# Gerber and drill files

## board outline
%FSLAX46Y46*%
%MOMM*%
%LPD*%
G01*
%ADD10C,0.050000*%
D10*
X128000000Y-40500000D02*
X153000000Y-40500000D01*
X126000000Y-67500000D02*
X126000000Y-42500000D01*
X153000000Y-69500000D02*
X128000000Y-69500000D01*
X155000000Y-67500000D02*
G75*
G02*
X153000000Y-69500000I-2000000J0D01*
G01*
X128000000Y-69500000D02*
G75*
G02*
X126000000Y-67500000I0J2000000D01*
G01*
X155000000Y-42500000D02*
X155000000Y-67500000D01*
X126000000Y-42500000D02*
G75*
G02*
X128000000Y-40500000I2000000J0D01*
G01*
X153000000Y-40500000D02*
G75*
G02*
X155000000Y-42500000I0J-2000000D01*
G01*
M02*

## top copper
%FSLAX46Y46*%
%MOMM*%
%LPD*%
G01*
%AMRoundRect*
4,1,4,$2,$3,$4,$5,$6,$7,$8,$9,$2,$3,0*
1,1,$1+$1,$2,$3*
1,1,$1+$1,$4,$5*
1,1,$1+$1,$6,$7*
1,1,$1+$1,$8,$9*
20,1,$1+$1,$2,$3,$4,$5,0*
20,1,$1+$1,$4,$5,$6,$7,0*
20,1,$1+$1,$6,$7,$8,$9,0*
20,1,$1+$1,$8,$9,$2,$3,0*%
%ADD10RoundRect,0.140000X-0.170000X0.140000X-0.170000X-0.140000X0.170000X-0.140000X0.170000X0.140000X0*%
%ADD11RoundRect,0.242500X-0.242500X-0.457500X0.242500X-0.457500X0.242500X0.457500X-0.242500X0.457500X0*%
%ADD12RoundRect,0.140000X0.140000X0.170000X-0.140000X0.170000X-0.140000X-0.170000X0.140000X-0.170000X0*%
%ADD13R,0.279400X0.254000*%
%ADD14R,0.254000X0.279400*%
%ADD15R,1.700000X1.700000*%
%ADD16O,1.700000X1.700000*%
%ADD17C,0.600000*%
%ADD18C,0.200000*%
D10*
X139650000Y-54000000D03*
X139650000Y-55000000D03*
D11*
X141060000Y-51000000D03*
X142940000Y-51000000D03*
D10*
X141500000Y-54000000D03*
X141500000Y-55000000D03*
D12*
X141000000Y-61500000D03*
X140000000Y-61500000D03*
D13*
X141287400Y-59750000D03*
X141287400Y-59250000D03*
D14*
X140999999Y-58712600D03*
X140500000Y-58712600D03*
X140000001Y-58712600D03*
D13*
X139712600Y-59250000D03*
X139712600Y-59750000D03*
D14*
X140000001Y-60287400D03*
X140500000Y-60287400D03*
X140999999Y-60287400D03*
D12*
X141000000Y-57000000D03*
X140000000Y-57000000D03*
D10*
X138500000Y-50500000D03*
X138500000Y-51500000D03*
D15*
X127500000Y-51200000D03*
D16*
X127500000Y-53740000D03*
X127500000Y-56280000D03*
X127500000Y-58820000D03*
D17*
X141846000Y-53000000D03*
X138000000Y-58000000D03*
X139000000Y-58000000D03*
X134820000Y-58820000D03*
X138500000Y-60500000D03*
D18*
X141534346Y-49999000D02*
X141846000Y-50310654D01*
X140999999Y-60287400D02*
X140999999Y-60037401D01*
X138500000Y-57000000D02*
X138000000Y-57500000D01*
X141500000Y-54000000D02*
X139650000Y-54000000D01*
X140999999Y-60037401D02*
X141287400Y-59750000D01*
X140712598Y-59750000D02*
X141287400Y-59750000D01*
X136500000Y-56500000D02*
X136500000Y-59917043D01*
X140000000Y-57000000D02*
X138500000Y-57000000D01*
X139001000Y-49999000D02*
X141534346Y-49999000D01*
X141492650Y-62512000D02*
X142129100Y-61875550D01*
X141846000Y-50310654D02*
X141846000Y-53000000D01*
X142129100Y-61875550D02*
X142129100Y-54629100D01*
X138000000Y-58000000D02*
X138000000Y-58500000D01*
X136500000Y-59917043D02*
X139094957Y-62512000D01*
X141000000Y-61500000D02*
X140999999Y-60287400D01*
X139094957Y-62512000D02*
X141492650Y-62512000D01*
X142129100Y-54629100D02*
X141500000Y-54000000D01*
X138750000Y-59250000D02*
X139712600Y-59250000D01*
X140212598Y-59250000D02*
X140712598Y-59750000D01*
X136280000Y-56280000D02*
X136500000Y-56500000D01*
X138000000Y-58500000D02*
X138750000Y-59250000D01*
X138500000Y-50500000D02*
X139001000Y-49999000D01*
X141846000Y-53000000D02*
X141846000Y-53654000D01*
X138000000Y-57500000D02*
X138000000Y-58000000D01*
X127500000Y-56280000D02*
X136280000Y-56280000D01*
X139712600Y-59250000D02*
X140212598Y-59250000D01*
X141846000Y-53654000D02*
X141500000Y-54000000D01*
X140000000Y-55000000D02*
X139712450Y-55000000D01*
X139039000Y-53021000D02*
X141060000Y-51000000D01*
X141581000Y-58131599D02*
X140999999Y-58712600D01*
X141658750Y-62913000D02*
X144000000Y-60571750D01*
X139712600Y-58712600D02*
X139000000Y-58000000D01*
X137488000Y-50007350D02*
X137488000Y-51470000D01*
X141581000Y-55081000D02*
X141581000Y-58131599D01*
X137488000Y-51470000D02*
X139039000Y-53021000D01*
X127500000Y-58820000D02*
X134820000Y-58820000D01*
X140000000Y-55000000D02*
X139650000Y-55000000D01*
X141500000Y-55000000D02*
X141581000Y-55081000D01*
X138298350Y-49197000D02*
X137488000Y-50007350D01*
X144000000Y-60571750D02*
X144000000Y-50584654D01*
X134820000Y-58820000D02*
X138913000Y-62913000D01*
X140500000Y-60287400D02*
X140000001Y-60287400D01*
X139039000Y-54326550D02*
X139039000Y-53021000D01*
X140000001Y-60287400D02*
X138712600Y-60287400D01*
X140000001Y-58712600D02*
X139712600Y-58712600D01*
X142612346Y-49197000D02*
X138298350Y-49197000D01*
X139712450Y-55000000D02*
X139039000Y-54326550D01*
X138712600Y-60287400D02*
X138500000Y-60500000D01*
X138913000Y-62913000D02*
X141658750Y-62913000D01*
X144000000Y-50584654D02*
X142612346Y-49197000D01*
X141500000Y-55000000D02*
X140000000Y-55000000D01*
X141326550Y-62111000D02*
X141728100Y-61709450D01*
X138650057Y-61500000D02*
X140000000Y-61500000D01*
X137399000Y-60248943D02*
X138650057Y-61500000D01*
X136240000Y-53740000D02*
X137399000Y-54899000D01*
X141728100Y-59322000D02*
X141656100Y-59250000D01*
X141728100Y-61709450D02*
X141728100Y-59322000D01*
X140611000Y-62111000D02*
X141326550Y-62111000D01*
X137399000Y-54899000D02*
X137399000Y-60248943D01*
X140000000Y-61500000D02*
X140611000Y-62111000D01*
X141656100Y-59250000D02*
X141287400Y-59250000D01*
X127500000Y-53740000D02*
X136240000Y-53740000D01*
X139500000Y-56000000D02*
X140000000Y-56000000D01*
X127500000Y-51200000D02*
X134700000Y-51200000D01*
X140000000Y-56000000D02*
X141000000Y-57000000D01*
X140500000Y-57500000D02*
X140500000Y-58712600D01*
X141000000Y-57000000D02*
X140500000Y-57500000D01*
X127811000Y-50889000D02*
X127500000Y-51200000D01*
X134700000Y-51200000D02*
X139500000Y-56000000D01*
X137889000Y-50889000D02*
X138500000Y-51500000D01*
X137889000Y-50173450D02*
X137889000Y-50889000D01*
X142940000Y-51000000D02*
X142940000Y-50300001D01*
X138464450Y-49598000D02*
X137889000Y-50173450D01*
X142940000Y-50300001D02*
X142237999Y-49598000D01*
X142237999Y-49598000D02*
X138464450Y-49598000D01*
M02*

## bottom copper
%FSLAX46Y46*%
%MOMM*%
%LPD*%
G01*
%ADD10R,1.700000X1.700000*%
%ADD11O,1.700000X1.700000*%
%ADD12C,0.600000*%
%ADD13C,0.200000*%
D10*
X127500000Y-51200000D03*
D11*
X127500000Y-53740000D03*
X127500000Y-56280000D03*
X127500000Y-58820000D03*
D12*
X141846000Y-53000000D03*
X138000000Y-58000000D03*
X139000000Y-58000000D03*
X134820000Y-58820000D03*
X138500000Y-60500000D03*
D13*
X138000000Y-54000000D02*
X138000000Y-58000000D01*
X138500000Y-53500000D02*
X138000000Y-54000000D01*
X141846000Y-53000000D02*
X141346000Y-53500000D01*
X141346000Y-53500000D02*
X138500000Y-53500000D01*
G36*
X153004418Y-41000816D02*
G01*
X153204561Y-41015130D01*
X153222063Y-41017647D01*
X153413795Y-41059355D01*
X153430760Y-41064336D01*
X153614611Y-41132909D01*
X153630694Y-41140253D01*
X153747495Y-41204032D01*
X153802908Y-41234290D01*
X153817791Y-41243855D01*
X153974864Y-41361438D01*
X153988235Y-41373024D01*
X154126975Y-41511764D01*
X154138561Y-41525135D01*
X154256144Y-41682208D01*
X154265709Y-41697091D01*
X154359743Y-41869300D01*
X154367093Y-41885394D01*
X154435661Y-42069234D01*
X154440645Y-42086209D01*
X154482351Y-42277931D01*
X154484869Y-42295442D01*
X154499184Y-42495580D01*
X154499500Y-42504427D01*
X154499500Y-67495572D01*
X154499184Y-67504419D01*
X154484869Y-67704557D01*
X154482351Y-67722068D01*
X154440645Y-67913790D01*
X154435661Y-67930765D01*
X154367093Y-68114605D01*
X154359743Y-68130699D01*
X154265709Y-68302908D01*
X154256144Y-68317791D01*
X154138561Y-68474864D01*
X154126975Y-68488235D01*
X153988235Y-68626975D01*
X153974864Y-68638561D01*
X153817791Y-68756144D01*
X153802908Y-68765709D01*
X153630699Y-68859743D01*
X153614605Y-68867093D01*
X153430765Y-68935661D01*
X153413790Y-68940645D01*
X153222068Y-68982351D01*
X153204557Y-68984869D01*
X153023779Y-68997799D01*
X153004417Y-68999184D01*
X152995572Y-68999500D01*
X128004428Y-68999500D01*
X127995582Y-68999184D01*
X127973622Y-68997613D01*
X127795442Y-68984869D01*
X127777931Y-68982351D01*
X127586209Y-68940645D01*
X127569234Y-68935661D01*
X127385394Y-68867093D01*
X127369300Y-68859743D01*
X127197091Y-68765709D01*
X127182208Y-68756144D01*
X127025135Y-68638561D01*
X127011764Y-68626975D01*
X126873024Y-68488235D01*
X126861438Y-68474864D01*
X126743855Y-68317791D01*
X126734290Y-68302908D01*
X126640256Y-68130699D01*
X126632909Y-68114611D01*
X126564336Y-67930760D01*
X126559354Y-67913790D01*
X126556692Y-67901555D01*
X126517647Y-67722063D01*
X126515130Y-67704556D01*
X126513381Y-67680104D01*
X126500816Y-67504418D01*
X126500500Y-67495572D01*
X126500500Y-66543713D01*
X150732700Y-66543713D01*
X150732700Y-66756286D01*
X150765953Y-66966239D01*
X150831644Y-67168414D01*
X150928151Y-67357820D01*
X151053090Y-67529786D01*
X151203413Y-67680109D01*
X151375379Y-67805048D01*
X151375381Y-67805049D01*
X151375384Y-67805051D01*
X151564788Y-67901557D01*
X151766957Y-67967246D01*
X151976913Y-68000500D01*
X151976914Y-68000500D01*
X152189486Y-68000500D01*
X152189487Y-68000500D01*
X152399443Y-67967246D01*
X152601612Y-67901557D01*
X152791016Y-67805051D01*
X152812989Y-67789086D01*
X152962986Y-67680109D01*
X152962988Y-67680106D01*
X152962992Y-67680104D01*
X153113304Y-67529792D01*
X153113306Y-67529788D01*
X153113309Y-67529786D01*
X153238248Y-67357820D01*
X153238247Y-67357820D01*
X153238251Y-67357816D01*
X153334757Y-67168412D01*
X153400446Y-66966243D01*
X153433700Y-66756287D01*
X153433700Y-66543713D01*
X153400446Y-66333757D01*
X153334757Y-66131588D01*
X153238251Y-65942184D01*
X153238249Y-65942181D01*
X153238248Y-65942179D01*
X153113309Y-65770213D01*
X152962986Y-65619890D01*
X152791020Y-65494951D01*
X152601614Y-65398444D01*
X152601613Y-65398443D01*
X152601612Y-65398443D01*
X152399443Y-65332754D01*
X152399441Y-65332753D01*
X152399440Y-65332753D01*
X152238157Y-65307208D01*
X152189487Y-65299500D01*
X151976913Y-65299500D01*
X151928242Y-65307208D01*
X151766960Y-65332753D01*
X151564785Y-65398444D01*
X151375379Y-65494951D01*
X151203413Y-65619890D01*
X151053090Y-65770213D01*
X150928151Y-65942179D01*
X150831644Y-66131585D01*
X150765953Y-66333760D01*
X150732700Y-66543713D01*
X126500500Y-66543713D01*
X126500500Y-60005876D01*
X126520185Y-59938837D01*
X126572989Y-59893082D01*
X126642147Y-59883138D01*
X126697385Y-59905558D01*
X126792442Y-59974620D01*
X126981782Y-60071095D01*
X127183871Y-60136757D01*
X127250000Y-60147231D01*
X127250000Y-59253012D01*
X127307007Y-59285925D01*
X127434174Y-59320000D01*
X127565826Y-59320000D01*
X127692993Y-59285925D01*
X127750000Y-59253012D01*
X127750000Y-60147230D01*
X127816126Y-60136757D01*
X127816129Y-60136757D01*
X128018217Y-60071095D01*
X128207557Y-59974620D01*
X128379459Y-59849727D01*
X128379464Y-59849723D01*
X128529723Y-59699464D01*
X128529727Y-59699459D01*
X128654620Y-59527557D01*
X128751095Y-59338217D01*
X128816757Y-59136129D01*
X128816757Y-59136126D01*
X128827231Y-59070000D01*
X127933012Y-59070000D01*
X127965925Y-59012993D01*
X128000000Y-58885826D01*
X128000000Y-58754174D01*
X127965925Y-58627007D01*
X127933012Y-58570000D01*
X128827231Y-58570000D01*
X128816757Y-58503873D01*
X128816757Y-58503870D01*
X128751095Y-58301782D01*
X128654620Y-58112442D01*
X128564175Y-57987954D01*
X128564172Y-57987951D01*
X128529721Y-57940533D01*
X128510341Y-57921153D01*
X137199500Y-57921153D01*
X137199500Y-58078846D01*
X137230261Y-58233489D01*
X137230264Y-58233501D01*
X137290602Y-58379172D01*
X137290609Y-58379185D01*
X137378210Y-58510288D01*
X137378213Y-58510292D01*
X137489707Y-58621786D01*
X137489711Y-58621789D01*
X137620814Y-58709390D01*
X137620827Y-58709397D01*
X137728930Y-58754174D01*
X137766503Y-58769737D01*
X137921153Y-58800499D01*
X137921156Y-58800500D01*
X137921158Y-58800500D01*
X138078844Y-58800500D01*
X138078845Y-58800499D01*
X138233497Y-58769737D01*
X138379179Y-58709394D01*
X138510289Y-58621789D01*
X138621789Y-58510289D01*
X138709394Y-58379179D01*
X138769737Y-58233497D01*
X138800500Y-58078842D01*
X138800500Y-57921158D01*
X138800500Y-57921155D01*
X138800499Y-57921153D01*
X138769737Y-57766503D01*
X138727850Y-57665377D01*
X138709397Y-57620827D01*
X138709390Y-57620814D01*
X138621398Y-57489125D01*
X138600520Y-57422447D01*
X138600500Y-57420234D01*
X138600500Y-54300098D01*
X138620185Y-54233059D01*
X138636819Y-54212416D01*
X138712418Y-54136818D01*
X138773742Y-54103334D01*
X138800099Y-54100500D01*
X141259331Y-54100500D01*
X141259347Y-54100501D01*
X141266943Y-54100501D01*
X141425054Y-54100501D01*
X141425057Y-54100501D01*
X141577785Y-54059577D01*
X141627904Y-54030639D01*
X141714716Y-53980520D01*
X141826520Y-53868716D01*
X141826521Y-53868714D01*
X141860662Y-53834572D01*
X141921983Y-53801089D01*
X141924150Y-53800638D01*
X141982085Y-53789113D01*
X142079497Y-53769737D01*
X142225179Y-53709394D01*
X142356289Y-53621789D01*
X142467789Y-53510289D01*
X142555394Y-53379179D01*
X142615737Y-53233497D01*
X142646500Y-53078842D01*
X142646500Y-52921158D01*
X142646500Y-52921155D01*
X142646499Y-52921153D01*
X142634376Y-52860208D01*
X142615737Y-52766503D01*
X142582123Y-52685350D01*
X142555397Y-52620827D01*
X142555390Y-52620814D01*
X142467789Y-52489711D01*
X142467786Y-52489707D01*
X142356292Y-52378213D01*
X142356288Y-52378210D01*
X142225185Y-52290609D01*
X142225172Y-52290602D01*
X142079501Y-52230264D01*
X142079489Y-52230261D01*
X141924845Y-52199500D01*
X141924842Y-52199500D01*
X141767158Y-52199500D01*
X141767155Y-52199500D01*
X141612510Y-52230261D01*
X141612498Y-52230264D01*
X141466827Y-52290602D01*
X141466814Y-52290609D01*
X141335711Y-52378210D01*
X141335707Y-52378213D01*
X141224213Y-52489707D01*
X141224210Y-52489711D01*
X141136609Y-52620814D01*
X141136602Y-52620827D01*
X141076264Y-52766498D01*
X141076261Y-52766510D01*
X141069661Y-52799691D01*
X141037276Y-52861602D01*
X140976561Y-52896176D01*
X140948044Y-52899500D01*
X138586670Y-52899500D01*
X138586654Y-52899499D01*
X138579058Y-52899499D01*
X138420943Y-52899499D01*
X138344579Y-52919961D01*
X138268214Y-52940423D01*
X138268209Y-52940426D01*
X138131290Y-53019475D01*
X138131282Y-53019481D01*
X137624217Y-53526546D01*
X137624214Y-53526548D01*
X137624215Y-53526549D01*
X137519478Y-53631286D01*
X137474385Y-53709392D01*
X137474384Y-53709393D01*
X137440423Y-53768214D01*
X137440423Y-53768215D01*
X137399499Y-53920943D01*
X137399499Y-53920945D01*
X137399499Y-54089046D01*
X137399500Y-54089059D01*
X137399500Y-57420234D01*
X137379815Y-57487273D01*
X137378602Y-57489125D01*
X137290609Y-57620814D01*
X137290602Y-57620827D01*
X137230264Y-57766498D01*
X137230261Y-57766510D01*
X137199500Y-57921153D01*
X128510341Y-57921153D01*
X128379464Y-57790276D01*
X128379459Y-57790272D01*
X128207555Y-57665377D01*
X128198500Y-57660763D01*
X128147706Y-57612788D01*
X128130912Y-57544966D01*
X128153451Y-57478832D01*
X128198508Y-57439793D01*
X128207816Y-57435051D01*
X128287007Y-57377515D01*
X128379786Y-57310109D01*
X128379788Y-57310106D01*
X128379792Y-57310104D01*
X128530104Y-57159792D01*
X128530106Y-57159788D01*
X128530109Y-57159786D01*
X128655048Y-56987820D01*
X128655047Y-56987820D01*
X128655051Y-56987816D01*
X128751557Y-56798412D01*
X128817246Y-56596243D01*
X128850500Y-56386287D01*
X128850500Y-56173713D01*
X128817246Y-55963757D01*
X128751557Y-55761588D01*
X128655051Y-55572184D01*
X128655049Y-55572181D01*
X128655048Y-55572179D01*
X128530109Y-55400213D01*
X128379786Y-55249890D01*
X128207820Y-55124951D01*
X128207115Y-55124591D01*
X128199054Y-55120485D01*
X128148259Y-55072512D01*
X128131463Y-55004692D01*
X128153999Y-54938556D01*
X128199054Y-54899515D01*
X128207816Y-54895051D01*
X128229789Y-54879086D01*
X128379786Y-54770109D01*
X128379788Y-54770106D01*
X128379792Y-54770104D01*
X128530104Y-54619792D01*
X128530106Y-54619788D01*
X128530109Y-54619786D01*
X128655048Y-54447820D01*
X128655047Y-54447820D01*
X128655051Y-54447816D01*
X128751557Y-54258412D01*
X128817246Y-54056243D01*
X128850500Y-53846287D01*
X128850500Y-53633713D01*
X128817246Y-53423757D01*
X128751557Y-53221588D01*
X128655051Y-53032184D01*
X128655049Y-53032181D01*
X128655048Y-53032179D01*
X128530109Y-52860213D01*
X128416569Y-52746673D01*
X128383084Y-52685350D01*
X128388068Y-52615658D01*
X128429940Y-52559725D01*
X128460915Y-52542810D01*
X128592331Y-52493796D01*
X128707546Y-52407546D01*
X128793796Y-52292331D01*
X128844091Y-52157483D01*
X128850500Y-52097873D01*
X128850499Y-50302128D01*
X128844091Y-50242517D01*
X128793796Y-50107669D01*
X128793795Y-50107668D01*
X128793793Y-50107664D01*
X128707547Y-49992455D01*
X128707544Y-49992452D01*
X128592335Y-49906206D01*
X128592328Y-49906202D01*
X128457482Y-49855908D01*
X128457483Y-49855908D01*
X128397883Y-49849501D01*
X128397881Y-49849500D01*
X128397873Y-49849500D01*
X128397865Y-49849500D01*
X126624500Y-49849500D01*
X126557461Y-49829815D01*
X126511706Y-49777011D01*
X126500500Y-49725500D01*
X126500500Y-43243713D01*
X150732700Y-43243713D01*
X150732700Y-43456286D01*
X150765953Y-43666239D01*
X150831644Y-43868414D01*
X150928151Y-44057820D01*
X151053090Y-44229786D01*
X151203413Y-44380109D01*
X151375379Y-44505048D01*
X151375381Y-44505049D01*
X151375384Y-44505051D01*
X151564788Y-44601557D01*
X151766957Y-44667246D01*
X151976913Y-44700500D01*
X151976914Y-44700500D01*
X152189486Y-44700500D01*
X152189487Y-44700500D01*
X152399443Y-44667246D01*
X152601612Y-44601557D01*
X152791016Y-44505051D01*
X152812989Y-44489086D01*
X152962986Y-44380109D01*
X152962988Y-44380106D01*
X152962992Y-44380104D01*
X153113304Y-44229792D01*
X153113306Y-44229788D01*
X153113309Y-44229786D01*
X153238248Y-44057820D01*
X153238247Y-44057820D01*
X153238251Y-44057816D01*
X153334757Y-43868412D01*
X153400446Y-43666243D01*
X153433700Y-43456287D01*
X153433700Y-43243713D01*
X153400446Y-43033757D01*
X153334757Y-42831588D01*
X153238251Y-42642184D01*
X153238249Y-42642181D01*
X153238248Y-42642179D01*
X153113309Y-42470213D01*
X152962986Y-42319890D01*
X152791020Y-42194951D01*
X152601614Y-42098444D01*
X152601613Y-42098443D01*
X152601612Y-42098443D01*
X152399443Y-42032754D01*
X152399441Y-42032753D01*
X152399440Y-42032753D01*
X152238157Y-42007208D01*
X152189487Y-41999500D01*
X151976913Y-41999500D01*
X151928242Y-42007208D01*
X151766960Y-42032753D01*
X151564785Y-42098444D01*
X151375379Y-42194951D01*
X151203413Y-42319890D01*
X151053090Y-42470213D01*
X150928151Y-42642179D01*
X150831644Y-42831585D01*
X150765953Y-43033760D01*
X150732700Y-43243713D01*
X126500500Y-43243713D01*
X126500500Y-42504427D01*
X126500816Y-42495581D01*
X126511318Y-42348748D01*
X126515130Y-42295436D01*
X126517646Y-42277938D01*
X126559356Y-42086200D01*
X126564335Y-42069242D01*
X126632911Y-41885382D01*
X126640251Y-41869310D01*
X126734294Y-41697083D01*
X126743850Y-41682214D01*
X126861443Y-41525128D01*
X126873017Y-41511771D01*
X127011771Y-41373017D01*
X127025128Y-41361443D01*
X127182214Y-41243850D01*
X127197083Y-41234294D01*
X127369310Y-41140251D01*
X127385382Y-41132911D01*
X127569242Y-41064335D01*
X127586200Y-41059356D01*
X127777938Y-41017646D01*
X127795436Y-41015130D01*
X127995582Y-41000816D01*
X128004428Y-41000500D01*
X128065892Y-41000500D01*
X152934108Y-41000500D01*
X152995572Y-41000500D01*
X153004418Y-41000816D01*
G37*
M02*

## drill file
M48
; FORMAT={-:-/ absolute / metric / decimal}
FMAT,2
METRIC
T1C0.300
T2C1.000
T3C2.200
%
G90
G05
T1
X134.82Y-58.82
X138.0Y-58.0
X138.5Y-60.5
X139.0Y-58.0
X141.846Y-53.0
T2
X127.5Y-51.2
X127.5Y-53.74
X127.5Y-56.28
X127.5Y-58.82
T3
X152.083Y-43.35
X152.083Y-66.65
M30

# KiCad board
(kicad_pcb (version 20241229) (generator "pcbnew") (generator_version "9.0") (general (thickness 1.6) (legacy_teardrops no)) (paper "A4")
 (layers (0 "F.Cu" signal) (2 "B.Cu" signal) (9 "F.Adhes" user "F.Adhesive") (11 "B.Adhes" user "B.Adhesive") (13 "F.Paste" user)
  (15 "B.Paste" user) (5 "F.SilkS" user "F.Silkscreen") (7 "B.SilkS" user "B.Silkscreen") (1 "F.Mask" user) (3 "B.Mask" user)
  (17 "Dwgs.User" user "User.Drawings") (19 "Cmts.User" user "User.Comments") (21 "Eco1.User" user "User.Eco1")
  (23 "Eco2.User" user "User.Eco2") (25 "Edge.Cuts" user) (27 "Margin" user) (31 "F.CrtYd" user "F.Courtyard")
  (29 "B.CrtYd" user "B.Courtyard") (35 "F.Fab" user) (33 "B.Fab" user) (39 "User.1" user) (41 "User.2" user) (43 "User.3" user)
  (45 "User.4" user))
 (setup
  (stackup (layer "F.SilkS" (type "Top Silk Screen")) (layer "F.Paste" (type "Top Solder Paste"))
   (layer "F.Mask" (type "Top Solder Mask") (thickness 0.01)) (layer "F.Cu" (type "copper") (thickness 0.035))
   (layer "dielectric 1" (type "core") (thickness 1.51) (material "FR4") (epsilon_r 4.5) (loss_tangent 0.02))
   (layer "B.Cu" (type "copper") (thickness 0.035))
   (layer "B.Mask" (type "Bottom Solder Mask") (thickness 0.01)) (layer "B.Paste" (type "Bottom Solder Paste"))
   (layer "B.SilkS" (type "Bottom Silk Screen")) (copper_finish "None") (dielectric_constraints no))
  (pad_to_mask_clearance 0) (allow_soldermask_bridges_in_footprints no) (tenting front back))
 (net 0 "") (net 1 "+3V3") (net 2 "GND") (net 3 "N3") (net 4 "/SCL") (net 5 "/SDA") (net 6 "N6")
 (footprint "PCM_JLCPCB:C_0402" (layer "F.Cu") (at 139.65 54.5 -90)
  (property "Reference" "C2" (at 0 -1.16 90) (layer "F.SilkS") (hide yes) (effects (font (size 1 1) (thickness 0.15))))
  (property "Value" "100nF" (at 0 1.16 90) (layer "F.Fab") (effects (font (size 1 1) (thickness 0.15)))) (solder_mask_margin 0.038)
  (pad "1" smd roundrect (at -0.5 0 270) (size 0.56 0.62) (layers "F.Cu" "F.Mask" "F.Paste") (roundrect_rratio 0.25) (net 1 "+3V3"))
  (pad "2" smd roundrect (at 0.5 0 270) (size 0.56 0.62) (layers "F.Cu" "F.Mask" "F.Paste") (roundrect_rratio 0.25) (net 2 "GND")))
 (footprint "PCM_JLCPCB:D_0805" (layer "F.Cu") (at 142 51)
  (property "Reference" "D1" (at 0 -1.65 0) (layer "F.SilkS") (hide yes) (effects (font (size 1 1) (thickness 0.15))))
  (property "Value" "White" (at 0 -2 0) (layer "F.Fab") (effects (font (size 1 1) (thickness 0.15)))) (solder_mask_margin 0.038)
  (pad "1" smd roundrect (at -0.94 0) (size 0.97 1.4) (layers "F.Cu" "F.Mask" "F.Paste") (roundrect_rratio 0.25) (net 2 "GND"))
  (pad "2" smd roundrect (at 0.94 0) (size 0.97 1.4) (layers "F.Cu" "F.Mask" "F.Paste") (roundrect_rratio 0.25) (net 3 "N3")))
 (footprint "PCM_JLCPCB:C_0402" (layer "F.Cu") (at 141.5 54.5 -90)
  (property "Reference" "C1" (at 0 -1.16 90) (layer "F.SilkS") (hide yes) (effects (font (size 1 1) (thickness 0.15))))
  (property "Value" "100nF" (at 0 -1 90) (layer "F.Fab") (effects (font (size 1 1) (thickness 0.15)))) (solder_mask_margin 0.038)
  (pad "1" smd roundrect (at -0.5 0 270) (size 0.56 0.62) (layers "F.Cu" "F.Mask" "F.Paste") (roundrect_rratio 0.25) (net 1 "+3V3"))
  (pad "2" smd roundrect (at 0.5 0 270) (size 0.56 0.62) (layers "F.Cu" "F.Mask" "F.Paste") (roundrect_rratio 0.25) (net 2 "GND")))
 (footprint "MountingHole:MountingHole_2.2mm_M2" (layer "F.Cu") (at 152.0832 66.65)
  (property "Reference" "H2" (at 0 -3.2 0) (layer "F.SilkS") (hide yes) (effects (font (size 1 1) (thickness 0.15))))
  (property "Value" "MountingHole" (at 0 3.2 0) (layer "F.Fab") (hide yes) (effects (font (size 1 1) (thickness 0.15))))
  (pad "" np_thru_hole circle (at 0 0) (size 2.2 2.2) (drill 2.2) (layers "*.Cu" "*.Mask")))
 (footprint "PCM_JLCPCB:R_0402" (layer "F.Cu") (at 140.5 61.5 180)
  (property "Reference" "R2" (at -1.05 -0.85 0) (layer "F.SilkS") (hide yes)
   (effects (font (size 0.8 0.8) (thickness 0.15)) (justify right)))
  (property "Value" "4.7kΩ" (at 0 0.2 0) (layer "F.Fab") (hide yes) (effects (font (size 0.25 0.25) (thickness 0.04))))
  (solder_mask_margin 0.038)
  (pad "1" smd roundrect (at -0.5 0 180) (size 0.56 0.62) (layers "F.Cu" "F.Mask" "F.Paste") (roundrect_rratio 0.25) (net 1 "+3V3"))
  (pad "2" smd roundrect (at 0.5 0 180) (size 0.56 0.62) (layers "F.Cu" "F.Mask" "F.Paste") (roundrect_rratio 0.25) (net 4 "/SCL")))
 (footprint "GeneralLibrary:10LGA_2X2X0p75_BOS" (layer "F.Cu") (at 140.5 59.5 180)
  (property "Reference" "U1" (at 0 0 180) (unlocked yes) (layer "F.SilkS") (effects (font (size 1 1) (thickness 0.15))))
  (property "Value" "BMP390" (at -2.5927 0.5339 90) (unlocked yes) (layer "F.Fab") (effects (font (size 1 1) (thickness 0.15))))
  (pad "1" smd rect (at -0.7874 -0.25 270) (size 0.254 0.2794) (layers "F.Cu" "F.Mask" "F.Paste") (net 1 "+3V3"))
  (pad "2" smd rect (at -0.7874 0.25 270) (size 0.254 0.2794) (layers "F.Cu" "F.Mask" "F.Paste") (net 4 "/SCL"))
  (pad "3" smd rect (at -0.499999 0.7874 180) (size 0.254 0.2794) (layers "F.Cu" "F.Mask" "F.Paste") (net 2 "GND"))
  (pad "4" smd rect (at 0 0.7874 180) (size 0.254 0.2794) (layers "F.Cu" "F.Mask" "F.Paste") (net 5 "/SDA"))
  (pad "5" smd rect (at 0.499999 0.7874 180) (size 0.254 0.2794) (layers "F.Cu" "F.Mask" "F.Paste") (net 2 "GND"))
  (pad "6" smd rect (at 0.7874 0.25 270) (size 0.254 0.2794) (layers "F.Cu" "F.Mask" "F.Paste") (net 1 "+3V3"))
  (pad "7" smd rect (at 0.7874 -0.25 270) (size 0.254 0.2794) (layers "F.Cu" "F.Mask" "F.Paste") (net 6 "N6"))
  (pad "8" smd rect (at 0.499999 -0.7874 180) (size 0.254 0.2794) (layers "F.Cu" "F.Mask" "F.Paste") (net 2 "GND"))
  (pad "9" smd rect (at 0 -0.7874 180) (size 0.254 0.2794) (layers "F.Cu" "F.Mask" "F.Paste") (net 2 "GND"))
  (pad "10" smd rect (at -0.499999 -0.7874 180) (size 0.254 0.2794) (layers "F.Cu" "F.Mask" "F.Paste") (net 1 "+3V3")))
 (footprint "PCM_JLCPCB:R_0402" (layer "F.Cu") (at 140.5 57 180)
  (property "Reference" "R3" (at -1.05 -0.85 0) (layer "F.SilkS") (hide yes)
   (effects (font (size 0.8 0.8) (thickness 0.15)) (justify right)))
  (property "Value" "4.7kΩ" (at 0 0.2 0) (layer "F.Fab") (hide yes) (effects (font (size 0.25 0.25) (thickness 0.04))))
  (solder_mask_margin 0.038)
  (pad "1" smd roundrect (at -0.5 0 180) (size 0.56 0.62) (layers "F.Cu" "F.Mask" "F.Paste") (roundrect_rratio 0.25) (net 5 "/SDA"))
  (pad "2" smd roundrect (at 0.5 0 180) (size 0.56 0.62) (layers "F.Cu" "F.Mask" "F.Paste") (roundrect_rratio 0.25) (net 1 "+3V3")))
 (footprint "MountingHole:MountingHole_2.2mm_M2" (layer "F.Cu") (at 152.0832 43.35)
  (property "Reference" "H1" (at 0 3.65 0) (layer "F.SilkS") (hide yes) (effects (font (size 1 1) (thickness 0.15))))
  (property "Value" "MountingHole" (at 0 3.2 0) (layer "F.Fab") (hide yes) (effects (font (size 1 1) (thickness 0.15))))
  (pad "" np_thru_hole circle (at 0 0) (size 2.2 2.2) (drill 2.2) (layers "*.Cu" "*.Mask")))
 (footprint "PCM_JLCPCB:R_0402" (layer "F.Cu") (at 138.5 51 -90)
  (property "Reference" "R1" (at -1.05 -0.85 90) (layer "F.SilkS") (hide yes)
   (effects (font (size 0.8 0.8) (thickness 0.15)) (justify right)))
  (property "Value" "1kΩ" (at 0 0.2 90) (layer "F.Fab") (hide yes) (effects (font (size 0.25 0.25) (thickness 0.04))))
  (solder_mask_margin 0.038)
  (pad "1" smd roundrect (at -0.5 0 270) (size 0.56 0.62) (layers "F.Cu" "F.Mask" "F.Paste") (roundrect_rratio 0.25) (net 1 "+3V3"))
  (pad "2" smd roundrect (at 0.5 0 270) (size 0.56 0.62) (layers "F.Cu" "F.Mask" "F.Paste") (roundrect_rratio 0.25) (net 3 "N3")))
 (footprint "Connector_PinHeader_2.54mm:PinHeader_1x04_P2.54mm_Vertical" (layer "B.Cu") (at 127.5 51.2 180)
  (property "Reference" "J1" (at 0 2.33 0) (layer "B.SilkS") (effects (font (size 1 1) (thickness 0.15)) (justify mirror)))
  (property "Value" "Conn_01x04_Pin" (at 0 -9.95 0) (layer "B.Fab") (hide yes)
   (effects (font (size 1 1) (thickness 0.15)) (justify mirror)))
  (pad "1" thru_hole rect (at 0 0 180) (size 1.7 1.7) (drill 1) (layers "*.Cu" "*.Mask") (remove_unused_layers no) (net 5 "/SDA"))
  (pad "2" thru_hole oval (at 0 -2.54 180) (size 1.7 1.7) (drill 1) (layers "*.Cu" "*.Mask") (remove_unused_layers no) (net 4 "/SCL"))
  (pad "3" thru_hole oval (at 0 -5.08 180) (size 1.7 1.7) (drill 1) (layers "*.Cu" "*.Mask") (remove_unused_layers no) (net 1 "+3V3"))
  (pad "4" thru_hole oval (at 0 -7.62 180) (size 1.7 1.7) (drill 1) (layers "*.Cu" "*.Mask") (remove_unused_layers no) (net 2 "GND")))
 (gr_line (start 128 40.5) (end 153 40.5) (stroke (width 0.05) (type default)) (layer "Edge.Cuts"))
 (gr_line (start 126 67.5) (end 126 42.5) (stroke (width 0.05) (type default)) (layer "Edge.Cuts"))
 (gr_line (start 153 69.5) (end 128 69.5) (stroke (width 0.05) (type default)) (layer "Edge.Cuts"))
 (gr_arc (start 155 67.5) (mid 154.414214 68.914214) (end 153 69.5) (stroke (width 0.05) (type default)) (layer "Edge.Cuts"))
 (gr_arc (start 128 69.5) (mid 126.585786 68.914214) (end 126 67.5) (stroke (width 0.05) (type default)) (layer "Edge.Cuts"))
 (gr_line (start 155 42.5) (end 155 67.5) (stroke (width 0.05) (type default)) (layer "Edge.Cuts"))
 (gr_arc (start 126 42.5) (mid 126.585786 41.085786) (end 128 40.5) (stroke (width 0.05) (type default)) (layer "Edge.Cuts"))
 (gr_arc (start 153 40.5) (mid 154.414214 41.085786) (end 155 42.5) (stroke (width 0.05) (type default)) (layer "Edge.Cuts"))
 (segment (start 141.534346 49.999) (end 141.846 50.310654) (width 0.2) (layer "F.Cu") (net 1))
 (segment (start 140.999999 60.2874) (end 140.999999 60.037401) (width 0.2) (layer "F.Cu") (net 1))
 (segment (start 138.5 57) (end 138 57.5) (width 0.2) (layer "F.Cu") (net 1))
 (segment (start 141.5 54) (end 139.65 54) (width 0.2) (layer "F.Cu") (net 1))
 (segment (start 140.999999 60.037401) (end 141.2874 59.75) (width 0.2) (layer "F.Cu") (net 1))
 (segment (start 140.712598 59.75) (end 141.2874 59.75) (width 0.2) (layer "F.Cu") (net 1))
 (segment (start 136.5 56.5) (end 136.5 59.917043) (width 0.2) (layer "F.Cu") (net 1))
 (segment (start 140 57) (end 138.5 57) (width 0.2) (layer "F.Cu") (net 1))
 (segment (start 139.001 49.999) (end 141.534346 49.999) (width 0.2) (layer "F.Cu") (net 1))
 (segment (start 141.49265 62.512) (end 142.1291 61.87555) (width 0.2) (layer "F.Cu") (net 1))
 (segment (start 141.846 50.310654) (end 141.846 53) (width 0.2) (layer "F.Cu") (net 1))
 (segment (start 142.1291 61.87555) (end 142.1291 54.6291) (width 0.2) (layer "F.Cu") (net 1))
 (segment (start 138 58) (end 138 58.5) (width 0.2) (layer "F.Cu") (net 1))
 (segment (start 136.5 59.917043) (end 139.094957 62.512) (width 0.2) (layer "F.Cu") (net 1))
 (segment (start 141 61.5) (end 140.999999 60.2874) (width 0.2) (layer "F.Cu") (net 1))
 (segment (start 139.094957 62.512) (end 141.49265 62.512) (width 0.2) (layer "F.Cu") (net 1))
 (segment (start 142.1291 54.6291) (end 141.5 54) (width 0.2) (layer "F.Cu") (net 1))
 (segment (start 138.75 59.25) (end 139.7126 59.25) (width 0.2) (layer "F.Cu") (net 1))
 (segment (start 140.212598 59.25) (end 140.712598 59.75) (width 0.2) (layer "F.Cu") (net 1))
 (segment (start 136.28 56.28) (end 136.5 56.5) (width 0.2) (layer "F.Cu") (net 1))
 (segment (start 138 58.5) (end 138.75 59.25) (width 0.2) (layer "F.Cu") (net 1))
 (segment (start 138.5 50.5) (end 139.001 49.999) (width 0.2) (layer "F.Cu") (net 1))
 (segment (start 141.846 53) (end 141.846 53.654) (width 0.2) (layer "F.Cu") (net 1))
 (segment (start 138 57.5) (end 138 58) (width 0.2) (layer "F.Cu") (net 1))
 (segment (start 127.5 56.28) (end 136.28 56.28) (width 0.2) (layer "F.Cu") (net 1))
 (segment (start 139.7126 59.25) (end 140.212598 59.25) (width 0.2) (layer "F.Cu") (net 1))
 (segment (start 141.846 53.654) (end 141.5 54) (width 0.2) (layer "F.Cu") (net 1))
 (via (at 141.846 53) (size 0.6) (drill 0.3) (layers "F.Cu" "B.Cu") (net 1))
 (via (at 138 58) (size 0.6) (drill 0.3) (layers "F.Cu" "B.Cu") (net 1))
 (segment (start 138 54) (end 138 58) (width 0.2) (layer "B.Cu") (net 1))
 (segment (start 138.5 53.5) (end 138 54) (width 0.2) (layer "B.Cu") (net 1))
 (segment (start 141.846 53) (end 141.346 53.5) (width 0.2) (layer "B.Cu") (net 1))
 (segment (start 141.346 53.5) (end 138.5 53.5) (width 0.2) (layer "B.Cu") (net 1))
 (segment (start 140 55) (end 139.71245 55) (width 0.2) (layer "F.Cu") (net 2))
 (segment (start 139.039 53.021) (end 141.06 51) (width 0.2) (layer "F.Cu") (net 2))
 (segment (start 141.581 58.131599) (end 140.999999 58.7126) (width 0.2) (layer "F.Cu") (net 2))
 (segment (start 141.65875 62.913) (end 144 60.57175) (width 0.2) (layer "F.Cu") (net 2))
 (segment (start 139.7126 58.7126) (end 139 58) (width 0.2) (layer "F.Cu") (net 2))
 (segment (start 137.488 50.00735) (end 137.488 51.47) (width 0.2) (layer "F.Cu") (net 2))
 (segment (start 141.581 55.081) (end 141.581 58.131599) (width 0.2) (layer "F.Cu") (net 2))
 (segment (start 137.488 51.47) (end 139.039 53.021) (width 0.2) (layer "F.Cu") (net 2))
 (segment (start 127.5 58.82) (end 134.82 58.82) (width 0.2) (layer "F.Cu") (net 2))
 (segment (start 140 55) (end 139.65 55) (width 0.2) (layer "F.Cu") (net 2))
 (segment (start 141.5 55) (end 141.581 55.081) (width 0.2) (layer "F.Cu") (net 2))
 (segment (start 138.29835 49.197) (end 137.488 50.00735) (width 0.2) (layer "F.Cu") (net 2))
 (segment (start 144 60.57175) (end 144 50.584654) (width 0.2) (layer "F.Cu") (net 2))
 (segment (start 134.82 58.82) (end 138.913 62.913) (width 0.2) (layer "F.Cu") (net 2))
 (segment (start 140.5 60.2874) (end 140.000001 60.2874) (width 0.2) (layer "F.Cu") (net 2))
 (segment (start 139.039 54.32655) (end 139.039 53.021) (width 0.2) (layer "F.Cu") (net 2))
 (segment (start 140.000001 60.2874) (end 138.7126 60.2874) (width 0.2) (layer "F.Cu") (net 2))
 (segment (start 140.000001 58.7126) (end 139.7126 58.7126) (width 0.2) (layer "F.Cu") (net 2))
 (segment (start 142.612346 49.197) (end 138.29835 49.197) (width 0.2) (layer "F.Cu") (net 2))
 (segment (start 139.71245 55) (end 139.039 54.32655) (width 0.2) (layer "F.Cu") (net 2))
 (segment (start 138.7126 60.2874) (end 138.5 60.5) (width 0.2) (layer "F.Cu") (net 2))
 (segment (start 138.913 62.913) (end 141.65875 62.913) (width 0.2) (layer "F.Cu") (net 2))
 (segment (start 144 50.584654) (end 142.612346 49.197) (width 0.2) (layer "F.Cu") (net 2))
 (segment (start 141.5 55) (end 140 55) (width 0.2) (layer "F.Cu") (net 2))
 (via (at 139 58) (size 0.6) (drill 0.3) (layers "F.Cu" "B.Cu") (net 2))
 (via (at 134.82 58.82) (size 0.6) (drill 0.3) (layers "F.Cu" "B.Cu") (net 2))
 (via (at 138.5 60.5) (size 0.6) (drill 0.3) (layers "F.Cu" "B.Cu") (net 2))
 (segment (start 141.32655 62.111) (end 141.7281 61.70945) (width 0.2) (layer "F.Cu") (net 4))
 (segment (start 138.650057 61.5) (end 140 61.5) (width 0.2) (layer "F.Cu") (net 4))
 (segment (start 137.399 60.248943) (end 138.650057 61.5) (width 0.2) (layer "F.Cu") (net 4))
 (segment (start 136.24 53.74) (end 137.399 54.899) (width 0.2) (layer "F.Cu") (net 4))
 (segment (start 141.7281 59.322) (end 141.6561 59.25) (width 0.2) (layer "F.Cu") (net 4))
 (segment (start 141.7281 61.70945) (end 141.7281 59.322) (width 0.2) (layer "F.Cu") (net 4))
 (segment (start 140.611 62.111) (end 141.32655 62.111) (width 0.2) (layer "F.Cu") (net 4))
 (segment (start 137.399 54.899) (end 137.399 60.248943) (width 0.2) (layer "F.Cu") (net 4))
 (segment (start 140 61.5) (end 140.611 62.111) (width 0.2) (layer "F.Cu") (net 4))
 (segment (start 141.6561 59.25) (end 141.2874 59.25) (width 0.2) (layer "F.Cu") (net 4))
 (segment (start 127.5 53.74) (end 136.24 53.74) (width 0.2) (layer "F.Cu") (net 4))
 (segment (start 139.5 56) (end 140 56) (width 0.2) (layer "F.Cu") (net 5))
 (segment (start 127.5 51.2) (end 134.7 51.2) (width 0.2) (layer "F.Cu") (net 5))
 (segment (start 140 56) (end 141 57) (width 0.2) (layer "F.Cu") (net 5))
 (segment (start 140.5 57.5) (end 140.5 58.7126) (width 0.2) (layer "F.Cu") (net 5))
 (segment (start 141 57) (end 140.5 57.5) (width 0.2) (layer "F.Cu") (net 5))
 (segment (start 127.811 50.889) (end 127.5 51.2) (width 0.2) (layer "F.Cu") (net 5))
 (segment (start 134.7 51.2) (end 139.5 56) (width 0.2) (layer "F.Cu") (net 5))
 (segment (start 137.889 50.889) (end 138.5 51.5) (width 0.2) (layer "F.Cu") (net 3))
 (segment (start 137.889 50.17345) (end 137.889 50.889) (width 0.2) (layer "F.Cu") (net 3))
 (segment (start 142.94 51) (end 142.94 50.300001) (width 0.2) (layer "F.Cu") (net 3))
 (segment (start 138.46445 49.598) (end 137.889 50.17345) (width 0.2) (layer "F.Cu") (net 3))
 (segment (start 142.94 50.300001) (end 142.237999 49.598) (width 0.2) (layer "F.Cu") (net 3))
 (segment (start 142.237999 49.598) (end 138.46445 49.598) (width 0.2) (layer "F.Cu") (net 3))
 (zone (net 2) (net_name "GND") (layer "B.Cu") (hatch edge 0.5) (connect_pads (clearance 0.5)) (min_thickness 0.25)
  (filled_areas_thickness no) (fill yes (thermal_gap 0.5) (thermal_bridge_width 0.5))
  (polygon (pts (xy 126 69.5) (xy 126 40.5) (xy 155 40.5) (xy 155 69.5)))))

